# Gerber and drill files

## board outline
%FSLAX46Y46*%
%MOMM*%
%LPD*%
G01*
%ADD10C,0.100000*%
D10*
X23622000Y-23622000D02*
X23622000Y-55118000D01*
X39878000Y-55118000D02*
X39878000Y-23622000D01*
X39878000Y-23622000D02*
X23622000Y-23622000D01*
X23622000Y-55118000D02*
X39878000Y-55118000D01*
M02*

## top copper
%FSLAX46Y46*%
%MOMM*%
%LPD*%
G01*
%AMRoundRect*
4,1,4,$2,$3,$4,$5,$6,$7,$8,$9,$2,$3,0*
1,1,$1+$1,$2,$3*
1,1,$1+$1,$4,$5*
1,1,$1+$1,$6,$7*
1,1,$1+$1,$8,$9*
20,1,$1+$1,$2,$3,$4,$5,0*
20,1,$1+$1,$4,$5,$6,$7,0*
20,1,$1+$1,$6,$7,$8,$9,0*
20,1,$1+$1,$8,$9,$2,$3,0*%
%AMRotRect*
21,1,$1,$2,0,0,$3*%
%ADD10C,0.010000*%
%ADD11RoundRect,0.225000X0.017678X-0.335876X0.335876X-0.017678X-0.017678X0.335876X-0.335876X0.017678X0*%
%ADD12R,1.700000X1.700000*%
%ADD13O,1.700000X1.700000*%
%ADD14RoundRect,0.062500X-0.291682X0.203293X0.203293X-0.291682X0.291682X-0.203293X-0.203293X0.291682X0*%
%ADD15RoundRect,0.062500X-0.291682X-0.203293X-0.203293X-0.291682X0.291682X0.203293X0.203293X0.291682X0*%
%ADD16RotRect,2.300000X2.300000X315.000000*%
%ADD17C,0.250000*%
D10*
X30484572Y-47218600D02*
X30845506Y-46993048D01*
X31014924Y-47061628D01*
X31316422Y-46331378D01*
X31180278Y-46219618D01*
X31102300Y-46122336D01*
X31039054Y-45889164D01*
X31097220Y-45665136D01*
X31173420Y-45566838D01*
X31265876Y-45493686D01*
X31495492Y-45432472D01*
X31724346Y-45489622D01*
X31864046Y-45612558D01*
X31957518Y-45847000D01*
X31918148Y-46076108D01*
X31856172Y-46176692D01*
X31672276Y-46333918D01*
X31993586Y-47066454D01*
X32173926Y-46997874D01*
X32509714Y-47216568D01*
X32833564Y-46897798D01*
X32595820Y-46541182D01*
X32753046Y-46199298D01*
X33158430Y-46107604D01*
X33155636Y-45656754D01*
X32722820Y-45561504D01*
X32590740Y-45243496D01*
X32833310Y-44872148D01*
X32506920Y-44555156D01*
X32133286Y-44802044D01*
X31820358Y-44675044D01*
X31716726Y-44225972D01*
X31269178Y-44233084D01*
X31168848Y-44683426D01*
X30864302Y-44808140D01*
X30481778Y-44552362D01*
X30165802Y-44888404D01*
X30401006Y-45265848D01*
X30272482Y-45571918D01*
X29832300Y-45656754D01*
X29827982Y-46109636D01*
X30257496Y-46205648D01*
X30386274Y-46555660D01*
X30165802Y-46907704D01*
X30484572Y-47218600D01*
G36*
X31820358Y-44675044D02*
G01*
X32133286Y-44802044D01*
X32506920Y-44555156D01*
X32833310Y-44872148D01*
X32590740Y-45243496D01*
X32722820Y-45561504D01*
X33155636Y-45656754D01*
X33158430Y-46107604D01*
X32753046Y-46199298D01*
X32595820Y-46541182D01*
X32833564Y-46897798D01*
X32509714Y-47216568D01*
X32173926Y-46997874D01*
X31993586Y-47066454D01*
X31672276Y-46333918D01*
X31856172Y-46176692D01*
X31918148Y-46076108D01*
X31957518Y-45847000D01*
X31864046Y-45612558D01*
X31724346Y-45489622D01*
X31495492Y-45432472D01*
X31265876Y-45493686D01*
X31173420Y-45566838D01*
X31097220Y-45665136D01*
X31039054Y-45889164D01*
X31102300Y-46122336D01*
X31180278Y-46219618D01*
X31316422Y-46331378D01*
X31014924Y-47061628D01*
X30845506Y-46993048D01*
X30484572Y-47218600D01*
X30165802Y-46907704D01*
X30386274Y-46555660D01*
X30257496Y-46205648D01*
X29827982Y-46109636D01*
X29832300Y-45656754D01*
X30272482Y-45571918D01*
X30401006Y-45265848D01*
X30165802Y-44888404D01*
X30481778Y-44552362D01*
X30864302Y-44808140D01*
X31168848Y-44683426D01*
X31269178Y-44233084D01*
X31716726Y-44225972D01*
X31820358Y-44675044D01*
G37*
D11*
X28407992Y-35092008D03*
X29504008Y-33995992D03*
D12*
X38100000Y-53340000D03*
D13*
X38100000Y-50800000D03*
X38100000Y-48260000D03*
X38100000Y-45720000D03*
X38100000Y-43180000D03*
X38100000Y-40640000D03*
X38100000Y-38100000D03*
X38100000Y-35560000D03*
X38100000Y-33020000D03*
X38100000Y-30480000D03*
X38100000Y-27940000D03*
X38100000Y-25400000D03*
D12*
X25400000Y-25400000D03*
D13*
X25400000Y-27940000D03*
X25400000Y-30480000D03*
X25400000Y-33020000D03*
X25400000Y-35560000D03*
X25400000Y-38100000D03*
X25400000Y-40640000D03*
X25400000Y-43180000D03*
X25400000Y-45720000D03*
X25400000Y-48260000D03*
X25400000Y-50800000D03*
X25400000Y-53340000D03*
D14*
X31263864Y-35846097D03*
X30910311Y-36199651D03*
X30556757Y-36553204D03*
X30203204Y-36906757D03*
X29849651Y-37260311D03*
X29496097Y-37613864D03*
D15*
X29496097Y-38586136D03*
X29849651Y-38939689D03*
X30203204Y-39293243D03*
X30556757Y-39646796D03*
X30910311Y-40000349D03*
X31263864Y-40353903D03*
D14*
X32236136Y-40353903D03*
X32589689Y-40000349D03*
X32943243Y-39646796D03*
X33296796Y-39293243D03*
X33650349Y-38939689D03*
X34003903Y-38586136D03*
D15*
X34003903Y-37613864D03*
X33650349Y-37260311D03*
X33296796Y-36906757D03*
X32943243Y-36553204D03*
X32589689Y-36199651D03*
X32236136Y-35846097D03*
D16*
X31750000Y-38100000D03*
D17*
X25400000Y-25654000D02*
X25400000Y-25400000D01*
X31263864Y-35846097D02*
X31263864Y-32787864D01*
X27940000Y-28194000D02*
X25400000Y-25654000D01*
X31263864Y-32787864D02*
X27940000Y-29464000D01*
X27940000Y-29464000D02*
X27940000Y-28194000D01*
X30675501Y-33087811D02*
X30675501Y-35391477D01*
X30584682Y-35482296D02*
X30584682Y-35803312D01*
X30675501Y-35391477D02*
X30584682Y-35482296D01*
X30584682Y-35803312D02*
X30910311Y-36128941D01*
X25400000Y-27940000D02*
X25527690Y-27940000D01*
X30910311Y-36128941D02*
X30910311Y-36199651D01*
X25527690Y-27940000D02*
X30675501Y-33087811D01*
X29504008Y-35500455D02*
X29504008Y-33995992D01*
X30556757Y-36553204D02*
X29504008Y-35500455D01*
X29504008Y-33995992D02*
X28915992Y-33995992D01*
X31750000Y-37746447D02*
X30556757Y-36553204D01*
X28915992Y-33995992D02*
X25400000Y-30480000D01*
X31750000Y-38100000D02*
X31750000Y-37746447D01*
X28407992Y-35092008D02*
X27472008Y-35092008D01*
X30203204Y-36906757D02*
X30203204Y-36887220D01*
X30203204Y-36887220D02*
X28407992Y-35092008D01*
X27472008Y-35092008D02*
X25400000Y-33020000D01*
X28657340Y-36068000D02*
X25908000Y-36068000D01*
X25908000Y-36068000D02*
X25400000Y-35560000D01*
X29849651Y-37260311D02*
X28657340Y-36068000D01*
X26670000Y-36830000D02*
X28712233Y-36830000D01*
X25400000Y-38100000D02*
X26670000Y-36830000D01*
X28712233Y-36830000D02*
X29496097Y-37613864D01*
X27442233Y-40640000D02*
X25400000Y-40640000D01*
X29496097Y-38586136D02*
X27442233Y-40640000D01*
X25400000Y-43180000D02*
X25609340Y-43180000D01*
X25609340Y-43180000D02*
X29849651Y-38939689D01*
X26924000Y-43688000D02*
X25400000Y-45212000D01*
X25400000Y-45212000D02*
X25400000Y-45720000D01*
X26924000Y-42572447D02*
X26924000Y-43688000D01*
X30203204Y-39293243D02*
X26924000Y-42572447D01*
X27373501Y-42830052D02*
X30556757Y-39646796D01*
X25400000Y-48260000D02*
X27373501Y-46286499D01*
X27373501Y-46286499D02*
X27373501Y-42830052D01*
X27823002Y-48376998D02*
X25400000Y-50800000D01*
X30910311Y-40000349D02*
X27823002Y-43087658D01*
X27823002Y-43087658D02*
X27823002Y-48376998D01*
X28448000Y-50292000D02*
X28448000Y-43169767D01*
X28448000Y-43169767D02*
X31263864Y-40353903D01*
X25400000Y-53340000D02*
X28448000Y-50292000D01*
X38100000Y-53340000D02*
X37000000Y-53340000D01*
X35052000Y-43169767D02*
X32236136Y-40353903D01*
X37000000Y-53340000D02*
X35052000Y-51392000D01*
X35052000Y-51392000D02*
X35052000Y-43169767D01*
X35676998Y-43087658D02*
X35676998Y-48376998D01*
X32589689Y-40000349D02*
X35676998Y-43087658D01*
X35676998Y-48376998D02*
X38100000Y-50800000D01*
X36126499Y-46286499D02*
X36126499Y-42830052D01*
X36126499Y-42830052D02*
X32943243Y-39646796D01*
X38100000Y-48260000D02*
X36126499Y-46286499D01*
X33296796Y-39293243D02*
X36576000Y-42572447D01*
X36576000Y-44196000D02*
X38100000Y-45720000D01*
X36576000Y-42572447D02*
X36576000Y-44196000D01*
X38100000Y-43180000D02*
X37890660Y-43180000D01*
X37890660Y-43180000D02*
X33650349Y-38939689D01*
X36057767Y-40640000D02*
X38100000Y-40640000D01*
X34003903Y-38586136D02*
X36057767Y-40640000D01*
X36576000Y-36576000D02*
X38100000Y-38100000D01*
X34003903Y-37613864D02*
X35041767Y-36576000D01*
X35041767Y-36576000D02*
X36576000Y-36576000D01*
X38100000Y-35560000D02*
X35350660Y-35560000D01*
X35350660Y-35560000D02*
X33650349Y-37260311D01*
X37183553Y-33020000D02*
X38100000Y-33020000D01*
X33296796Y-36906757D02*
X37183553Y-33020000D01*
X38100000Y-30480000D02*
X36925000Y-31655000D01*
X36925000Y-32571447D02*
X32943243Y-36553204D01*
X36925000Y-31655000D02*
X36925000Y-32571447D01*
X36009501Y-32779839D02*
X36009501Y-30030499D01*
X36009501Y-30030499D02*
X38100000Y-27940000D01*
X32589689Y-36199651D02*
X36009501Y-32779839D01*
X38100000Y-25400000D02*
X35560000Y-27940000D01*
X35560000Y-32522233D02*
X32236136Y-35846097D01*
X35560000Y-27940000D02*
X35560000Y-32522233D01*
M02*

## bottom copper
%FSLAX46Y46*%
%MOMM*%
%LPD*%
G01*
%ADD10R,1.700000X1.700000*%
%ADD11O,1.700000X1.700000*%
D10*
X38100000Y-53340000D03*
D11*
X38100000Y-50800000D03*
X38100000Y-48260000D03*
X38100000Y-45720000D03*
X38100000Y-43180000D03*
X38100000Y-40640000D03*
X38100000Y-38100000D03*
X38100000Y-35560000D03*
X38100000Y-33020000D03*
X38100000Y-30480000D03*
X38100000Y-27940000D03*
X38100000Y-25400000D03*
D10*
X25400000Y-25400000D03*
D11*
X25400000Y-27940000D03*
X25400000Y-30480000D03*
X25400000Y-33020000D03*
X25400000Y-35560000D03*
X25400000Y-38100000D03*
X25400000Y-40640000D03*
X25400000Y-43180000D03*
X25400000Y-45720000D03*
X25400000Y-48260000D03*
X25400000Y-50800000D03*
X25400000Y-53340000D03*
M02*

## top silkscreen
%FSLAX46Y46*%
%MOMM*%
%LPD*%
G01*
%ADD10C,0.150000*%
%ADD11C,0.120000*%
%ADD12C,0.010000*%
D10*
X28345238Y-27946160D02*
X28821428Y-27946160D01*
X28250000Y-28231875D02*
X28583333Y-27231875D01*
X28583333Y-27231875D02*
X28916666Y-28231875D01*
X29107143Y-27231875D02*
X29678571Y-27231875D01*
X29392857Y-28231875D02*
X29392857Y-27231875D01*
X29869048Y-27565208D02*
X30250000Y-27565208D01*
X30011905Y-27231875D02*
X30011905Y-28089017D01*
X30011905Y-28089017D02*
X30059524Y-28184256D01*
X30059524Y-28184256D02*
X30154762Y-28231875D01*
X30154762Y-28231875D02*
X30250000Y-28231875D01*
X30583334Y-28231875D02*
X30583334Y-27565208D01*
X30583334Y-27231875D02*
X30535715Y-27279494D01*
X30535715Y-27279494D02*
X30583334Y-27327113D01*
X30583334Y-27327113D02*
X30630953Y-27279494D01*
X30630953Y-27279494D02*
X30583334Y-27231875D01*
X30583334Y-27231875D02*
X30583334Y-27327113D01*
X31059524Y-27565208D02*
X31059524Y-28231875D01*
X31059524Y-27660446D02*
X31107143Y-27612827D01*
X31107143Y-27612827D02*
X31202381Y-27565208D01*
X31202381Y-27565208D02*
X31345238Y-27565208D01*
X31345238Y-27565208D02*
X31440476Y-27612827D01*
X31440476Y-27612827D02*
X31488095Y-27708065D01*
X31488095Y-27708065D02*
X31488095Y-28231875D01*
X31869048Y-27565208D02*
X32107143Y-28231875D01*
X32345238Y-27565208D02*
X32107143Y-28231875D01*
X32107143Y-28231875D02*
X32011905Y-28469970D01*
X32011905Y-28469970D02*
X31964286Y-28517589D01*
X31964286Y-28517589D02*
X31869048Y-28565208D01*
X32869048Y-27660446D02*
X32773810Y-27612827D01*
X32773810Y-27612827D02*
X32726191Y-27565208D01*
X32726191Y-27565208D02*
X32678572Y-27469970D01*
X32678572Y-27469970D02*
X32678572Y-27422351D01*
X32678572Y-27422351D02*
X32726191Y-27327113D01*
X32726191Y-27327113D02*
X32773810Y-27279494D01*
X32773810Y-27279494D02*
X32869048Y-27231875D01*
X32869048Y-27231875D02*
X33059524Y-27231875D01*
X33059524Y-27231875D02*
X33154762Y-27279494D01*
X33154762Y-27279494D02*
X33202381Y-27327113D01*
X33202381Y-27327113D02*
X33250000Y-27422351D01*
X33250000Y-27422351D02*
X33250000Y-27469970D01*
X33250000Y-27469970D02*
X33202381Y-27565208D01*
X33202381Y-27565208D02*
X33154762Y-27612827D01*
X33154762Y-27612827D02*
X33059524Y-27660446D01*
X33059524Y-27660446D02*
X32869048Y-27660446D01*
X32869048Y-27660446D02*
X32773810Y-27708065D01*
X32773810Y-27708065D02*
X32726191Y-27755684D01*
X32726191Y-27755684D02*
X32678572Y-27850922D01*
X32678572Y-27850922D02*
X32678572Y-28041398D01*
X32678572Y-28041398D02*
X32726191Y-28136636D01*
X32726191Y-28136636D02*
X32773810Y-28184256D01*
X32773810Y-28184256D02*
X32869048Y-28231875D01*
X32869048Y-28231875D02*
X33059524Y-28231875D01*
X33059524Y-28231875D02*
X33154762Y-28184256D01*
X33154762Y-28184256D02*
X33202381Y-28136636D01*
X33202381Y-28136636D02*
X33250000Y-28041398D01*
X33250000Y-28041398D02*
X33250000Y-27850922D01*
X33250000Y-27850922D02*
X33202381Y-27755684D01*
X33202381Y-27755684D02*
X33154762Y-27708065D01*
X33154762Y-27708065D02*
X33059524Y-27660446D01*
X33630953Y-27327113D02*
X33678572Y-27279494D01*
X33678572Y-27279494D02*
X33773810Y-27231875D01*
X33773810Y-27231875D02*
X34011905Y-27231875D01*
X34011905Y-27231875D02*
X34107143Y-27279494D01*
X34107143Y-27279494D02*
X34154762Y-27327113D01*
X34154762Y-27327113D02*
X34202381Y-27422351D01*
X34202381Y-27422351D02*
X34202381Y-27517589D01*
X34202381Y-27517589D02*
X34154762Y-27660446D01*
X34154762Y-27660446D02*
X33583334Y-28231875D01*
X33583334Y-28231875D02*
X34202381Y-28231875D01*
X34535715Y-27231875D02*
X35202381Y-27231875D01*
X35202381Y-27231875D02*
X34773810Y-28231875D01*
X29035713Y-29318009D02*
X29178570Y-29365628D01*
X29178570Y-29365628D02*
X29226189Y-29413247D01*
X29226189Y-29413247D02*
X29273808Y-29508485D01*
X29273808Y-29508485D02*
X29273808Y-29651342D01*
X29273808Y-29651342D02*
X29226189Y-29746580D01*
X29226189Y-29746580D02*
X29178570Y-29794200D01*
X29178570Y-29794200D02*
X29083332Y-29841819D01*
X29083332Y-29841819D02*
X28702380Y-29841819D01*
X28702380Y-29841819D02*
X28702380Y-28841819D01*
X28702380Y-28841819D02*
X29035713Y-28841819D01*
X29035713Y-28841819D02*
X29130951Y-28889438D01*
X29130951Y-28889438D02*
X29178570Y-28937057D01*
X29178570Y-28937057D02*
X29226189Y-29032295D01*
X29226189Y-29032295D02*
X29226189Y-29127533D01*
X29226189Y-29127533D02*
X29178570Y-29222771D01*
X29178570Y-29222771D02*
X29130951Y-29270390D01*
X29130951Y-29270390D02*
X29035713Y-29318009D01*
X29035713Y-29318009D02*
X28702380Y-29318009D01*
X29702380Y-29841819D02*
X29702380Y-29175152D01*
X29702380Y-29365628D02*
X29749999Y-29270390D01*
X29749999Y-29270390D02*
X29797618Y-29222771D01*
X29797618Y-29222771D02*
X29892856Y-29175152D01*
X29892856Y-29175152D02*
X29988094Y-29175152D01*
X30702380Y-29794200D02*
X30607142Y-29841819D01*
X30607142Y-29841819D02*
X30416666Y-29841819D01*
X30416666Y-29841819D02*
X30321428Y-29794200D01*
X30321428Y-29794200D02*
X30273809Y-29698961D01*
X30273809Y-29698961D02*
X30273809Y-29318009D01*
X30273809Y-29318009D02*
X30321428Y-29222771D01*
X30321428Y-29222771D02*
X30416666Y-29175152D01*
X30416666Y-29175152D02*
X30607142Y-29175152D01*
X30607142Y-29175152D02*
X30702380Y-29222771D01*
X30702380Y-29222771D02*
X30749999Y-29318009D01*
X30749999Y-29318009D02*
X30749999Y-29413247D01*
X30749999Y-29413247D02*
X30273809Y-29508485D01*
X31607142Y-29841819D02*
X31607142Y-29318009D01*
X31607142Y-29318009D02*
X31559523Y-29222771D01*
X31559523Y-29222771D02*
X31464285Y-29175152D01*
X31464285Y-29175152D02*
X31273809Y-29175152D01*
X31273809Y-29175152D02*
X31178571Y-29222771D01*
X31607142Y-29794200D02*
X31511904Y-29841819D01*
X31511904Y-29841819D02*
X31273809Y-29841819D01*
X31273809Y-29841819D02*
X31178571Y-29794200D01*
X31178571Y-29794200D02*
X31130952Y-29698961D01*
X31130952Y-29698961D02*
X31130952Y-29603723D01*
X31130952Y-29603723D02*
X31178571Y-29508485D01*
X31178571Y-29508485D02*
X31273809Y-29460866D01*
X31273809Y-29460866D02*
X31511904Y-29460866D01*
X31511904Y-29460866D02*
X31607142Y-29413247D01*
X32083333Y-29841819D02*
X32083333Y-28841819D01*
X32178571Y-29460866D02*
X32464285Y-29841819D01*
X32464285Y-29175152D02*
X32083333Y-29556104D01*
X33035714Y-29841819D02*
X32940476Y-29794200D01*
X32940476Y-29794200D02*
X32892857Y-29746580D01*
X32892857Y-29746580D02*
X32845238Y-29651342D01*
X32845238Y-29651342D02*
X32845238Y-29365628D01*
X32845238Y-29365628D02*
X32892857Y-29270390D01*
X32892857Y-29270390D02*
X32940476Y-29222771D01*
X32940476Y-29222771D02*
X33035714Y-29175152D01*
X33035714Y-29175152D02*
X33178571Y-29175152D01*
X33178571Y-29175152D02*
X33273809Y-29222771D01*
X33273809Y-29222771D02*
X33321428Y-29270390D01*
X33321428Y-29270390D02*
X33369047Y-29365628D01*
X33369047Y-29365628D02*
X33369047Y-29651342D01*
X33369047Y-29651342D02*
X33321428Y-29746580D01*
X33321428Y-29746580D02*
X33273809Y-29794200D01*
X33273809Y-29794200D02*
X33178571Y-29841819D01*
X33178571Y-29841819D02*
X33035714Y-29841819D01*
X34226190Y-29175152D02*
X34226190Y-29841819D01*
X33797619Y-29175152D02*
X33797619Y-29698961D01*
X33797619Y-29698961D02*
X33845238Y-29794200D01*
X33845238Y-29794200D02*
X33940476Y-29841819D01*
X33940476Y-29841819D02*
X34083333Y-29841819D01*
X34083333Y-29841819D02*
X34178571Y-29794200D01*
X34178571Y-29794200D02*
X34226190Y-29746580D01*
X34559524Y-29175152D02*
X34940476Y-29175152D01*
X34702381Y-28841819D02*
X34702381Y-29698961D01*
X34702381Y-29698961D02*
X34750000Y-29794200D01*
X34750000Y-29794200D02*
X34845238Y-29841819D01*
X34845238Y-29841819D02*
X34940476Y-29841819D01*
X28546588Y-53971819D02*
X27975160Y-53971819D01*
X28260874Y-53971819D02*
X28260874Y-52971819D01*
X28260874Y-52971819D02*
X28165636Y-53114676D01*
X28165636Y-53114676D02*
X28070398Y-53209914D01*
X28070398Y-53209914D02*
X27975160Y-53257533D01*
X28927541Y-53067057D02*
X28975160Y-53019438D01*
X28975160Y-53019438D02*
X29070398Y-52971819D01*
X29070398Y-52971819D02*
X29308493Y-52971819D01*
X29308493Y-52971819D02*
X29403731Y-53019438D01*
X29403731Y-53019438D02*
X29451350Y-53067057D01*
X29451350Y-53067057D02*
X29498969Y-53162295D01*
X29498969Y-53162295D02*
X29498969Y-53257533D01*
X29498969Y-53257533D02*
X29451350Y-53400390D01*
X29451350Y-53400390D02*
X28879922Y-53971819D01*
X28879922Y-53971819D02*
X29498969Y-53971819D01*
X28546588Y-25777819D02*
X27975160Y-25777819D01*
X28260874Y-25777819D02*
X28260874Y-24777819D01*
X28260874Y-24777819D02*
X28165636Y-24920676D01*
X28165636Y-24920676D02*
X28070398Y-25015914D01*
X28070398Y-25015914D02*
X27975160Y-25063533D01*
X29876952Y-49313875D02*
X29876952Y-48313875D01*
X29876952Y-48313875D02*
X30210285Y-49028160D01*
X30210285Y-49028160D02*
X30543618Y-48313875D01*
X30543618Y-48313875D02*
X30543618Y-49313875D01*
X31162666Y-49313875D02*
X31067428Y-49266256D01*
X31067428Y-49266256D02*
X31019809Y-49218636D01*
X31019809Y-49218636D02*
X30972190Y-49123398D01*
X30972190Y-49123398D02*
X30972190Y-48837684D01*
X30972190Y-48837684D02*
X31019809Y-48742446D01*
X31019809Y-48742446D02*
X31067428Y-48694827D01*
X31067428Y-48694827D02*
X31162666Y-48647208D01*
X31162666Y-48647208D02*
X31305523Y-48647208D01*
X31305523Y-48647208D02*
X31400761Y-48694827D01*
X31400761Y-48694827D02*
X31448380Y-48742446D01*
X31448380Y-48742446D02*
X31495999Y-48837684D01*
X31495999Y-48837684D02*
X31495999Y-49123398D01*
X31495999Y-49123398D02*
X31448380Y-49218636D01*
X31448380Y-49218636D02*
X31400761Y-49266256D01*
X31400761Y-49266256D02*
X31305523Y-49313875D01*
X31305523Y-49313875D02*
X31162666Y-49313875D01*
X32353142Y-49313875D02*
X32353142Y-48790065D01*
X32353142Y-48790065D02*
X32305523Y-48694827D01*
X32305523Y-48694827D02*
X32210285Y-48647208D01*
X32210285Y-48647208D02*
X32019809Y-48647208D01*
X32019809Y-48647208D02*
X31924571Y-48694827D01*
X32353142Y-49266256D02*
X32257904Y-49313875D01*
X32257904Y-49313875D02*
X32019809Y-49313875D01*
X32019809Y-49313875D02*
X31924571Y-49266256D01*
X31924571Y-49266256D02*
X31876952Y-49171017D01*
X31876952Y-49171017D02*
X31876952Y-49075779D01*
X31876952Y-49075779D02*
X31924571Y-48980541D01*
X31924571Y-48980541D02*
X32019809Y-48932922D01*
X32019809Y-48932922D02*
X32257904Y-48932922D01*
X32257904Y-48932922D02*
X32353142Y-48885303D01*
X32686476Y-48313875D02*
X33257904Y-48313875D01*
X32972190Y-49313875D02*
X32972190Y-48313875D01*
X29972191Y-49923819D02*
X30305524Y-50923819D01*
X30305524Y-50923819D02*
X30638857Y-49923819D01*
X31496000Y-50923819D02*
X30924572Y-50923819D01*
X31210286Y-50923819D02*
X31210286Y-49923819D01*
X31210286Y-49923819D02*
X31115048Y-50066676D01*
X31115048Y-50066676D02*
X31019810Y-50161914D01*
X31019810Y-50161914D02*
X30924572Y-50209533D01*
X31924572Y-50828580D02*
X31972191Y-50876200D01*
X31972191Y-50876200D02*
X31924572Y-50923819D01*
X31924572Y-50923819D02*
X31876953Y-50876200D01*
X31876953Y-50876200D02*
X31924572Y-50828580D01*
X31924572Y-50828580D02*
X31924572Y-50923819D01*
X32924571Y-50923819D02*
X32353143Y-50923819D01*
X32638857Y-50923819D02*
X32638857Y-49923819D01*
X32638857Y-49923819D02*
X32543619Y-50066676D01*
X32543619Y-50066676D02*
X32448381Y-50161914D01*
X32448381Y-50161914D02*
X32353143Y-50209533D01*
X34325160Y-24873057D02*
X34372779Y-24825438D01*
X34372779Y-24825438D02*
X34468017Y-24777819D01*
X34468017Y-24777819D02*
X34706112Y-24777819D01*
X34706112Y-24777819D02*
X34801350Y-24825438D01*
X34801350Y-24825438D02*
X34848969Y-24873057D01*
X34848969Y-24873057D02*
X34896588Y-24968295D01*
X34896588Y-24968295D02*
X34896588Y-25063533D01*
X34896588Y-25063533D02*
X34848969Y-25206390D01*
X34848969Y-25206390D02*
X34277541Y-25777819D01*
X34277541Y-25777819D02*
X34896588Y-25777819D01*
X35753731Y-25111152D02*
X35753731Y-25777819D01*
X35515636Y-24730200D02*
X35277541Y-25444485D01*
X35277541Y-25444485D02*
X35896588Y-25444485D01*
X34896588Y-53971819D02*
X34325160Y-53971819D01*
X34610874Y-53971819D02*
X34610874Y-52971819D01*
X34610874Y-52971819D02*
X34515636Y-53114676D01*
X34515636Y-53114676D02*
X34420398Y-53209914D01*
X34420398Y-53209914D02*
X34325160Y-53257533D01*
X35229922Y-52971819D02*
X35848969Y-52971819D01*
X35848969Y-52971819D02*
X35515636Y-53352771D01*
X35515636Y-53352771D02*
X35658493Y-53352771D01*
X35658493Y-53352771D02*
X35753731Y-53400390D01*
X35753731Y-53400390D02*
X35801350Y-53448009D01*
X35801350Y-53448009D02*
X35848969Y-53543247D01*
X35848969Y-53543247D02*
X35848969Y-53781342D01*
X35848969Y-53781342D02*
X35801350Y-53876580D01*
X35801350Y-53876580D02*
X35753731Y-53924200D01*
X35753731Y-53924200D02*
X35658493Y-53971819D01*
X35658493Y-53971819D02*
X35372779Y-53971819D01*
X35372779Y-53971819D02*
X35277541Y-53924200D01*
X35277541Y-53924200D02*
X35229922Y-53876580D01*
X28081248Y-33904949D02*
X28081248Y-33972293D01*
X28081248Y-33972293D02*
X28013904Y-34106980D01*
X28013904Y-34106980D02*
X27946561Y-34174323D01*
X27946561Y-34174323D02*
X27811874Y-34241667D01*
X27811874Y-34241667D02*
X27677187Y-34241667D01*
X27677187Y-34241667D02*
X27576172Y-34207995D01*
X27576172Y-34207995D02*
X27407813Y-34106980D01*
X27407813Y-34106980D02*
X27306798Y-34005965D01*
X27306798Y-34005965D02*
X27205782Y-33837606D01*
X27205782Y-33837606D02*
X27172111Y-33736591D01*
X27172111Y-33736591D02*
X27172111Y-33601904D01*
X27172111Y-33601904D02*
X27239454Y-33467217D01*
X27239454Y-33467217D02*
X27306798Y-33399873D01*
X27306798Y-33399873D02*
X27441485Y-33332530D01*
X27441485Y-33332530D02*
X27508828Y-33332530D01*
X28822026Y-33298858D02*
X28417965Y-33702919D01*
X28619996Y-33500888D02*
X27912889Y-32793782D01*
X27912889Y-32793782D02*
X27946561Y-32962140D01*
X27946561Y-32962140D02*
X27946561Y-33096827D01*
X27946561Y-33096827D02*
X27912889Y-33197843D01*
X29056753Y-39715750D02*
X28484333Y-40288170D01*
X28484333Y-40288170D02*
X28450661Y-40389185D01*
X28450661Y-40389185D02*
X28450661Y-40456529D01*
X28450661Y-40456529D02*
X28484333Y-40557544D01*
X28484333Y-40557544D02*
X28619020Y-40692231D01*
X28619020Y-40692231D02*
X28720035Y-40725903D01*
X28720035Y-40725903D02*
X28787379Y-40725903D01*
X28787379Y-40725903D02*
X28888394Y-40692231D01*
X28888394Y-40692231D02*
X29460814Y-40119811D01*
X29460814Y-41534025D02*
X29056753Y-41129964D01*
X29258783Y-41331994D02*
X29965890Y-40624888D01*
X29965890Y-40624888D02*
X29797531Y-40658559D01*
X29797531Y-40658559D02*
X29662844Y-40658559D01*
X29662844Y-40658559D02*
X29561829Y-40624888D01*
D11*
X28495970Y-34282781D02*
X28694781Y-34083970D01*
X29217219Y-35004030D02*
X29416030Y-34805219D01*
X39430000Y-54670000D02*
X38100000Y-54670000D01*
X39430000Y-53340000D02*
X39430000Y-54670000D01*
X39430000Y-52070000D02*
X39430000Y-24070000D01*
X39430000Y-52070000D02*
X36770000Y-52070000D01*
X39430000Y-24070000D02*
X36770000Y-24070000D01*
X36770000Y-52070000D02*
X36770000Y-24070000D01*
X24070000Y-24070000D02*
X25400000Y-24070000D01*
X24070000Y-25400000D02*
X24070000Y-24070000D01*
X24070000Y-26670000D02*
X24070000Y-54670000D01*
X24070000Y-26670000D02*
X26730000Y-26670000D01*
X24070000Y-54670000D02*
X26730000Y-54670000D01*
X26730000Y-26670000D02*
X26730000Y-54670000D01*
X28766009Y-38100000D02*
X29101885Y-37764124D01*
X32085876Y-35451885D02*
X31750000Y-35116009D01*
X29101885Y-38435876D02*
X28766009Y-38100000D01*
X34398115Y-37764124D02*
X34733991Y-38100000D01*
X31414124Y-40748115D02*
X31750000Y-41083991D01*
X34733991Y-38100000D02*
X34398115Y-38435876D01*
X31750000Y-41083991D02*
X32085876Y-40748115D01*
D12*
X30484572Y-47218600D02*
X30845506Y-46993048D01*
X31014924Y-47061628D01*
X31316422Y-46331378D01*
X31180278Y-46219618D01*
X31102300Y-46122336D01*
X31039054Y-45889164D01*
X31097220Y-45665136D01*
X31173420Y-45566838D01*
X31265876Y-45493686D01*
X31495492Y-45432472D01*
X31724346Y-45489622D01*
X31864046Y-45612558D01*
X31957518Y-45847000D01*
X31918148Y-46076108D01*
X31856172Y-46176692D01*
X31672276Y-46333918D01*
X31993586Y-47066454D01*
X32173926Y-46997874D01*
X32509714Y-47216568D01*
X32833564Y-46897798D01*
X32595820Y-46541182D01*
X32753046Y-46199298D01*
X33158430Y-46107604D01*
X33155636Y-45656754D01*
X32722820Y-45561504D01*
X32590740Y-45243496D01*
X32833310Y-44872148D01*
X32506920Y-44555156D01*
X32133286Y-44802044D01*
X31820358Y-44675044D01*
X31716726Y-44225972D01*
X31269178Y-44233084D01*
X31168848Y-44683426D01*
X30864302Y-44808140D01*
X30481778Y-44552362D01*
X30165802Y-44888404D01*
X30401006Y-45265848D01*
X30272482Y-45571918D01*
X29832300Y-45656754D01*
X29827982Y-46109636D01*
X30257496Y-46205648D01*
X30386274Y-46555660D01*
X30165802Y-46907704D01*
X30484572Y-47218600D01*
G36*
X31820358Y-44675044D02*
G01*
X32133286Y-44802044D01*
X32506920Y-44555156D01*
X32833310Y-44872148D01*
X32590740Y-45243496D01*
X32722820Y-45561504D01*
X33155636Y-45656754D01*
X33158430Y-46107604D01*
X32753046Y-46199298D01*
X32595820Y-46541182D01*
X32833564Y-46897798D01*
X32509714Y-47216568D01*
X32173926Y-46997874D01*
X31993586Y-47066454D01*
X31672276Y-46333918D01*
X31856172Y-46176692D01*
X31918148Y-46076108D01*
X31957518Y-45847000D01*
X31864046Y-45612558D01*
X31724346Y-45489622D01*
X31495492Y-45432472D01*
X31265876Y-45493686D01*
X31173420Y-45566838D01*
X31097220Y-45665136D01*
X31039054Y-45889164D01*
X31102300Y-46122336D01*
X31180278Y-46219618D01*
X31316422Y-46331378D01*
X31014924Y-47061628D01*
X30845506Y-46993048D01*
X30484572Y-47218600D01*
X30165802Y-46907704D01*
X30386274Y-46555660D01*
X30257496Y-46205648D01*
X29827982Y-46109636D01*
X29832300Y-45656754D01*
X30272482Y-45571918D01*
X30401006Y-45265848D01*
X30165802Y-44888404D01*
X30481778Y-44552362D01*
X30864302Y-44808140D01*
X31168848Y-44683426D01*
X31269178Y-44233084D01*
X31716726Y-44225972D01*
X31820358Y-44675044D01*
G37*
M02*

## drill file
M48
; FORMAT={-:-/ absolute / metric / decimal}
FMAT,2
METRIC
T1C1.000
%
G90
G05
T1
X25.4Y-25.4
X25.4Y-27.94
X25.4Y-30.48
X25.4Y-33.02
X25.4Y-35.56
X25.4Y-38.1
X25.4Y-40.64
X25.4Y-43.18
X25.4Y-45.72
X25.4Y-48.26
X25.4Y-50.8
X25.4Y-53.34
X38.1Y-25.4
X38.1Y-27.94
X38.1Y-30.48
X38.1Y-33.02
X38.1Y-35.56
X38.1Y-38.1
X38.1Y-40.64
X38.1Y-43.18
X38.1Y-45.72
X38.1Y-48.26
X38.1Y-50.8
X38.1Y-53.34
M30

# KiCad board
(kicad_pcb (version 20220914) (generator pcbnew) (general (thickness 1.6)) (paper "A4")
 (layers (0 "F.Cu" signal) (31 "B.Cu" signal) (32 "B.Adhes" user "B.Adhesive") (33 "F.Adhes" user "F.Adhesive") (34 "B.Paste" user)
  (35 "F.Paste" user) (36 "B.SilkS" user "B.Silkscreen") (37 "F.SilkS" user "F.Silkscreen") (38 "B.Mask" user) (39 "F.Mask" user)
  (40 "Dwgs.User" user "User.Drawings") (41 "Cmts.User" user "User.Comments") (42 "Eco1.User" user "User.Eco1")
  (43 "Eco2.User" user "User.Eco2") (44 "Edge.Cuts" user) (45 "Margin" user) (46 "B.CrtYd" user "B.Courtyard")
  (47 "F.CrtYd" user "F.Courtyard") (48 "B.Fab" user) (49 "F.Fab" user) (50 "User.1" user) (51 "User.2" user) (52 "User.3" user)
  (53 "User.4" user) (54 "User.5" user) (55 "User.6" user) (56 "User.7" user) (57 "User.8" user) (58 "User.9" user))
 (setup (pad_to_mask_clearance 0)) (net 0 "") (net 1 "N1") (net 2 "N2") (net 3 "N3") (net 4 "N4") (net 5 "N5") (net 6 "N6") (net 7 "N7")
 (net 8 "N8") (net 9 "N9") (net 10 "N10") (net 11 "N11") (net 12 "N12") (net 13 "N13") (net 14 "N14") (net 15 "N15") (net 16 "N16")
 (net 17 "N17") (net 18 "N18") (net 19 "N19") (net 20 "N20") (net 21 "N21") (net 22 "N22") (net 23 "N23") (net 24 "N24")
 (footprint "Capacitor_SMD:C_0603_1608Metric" (layer "F.Cu") (at 28.956 34.544 45)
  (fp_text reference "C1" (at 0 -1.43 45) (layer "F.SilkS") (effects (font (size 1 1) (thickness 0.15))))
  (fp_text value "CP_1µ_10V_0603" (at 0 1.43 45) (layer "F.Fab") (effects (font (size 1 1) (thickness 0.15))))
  (fp_line (start -0.14058 -0.51) (end 0.14058 -0.51) (stroke (width 0.12) (type solid)) (layer "F.SilkS"))
  (fp_line (start -0.14058 0.51) (end 0.14058 0.51) (stroke (width 0.12) (type solid)) (layer "F.SilkS"))
  (pad "1" smd roundrect (at -0.775 0 45) (size 0.9 0.95) (layers "F.Cu" "F.Paste" "F.Mask") (roundrect_rratio 0.25) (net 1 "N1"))
  (pad "2" smd roundrect (at 0.775 0 45) (size 0.9 0.95) (layers "F.Cu" "F.Paste" "F.Mask") (roundrect_rratio 0.25) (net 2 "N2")))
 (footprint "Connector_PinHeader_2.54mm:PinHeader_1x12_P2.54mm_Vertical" (layer "F.Cu") (at 38.1 53.34 180)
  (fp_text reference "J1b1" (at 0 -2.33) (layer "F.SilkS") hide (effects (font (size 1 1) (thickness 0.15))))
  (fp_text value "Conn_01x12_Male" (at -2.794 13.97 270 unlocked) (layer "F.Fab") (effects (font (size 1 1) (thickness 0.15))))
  (fp_line (start -1.33 -1.33) (end 0 -1.33) (stroke (width 0.12) (type solid)) (layer "F.SilkS"))
  (fp_line (start -1.33 0) (end -1.33 -1.33) (stroke (width 0.12) (type solid)) (layer "F.SilkS"))
  (fp_line (start -1.33 1.27) (end -1.33 29.27) (stroke (width 0.12) (type solid)) (layer "F.SilkS"))
  (fp_line (start -1.33 1.27) (end 1.33 1.27) (stroke (width 0.12) (type solid)) (layer "F.SilkS"))
  (fp_line (start -1.33 29.27) (end 1.33 29.27) (stroke (width 0.12) (type solid)) (layer "F.SilkS"))
  (fp_line (start 1.33 1.27) (end 1.33 29.27) (stroke (width 0.12) (type solid)) (layer "F.SilkS"))
  (pad "1" thru_hole rect (at 0 0 180) (size 1.7 1.7) (drill 1) (layers *.Cu *.Mask) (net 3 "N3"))
  (pad "2" thru_hole oval (at 0 2.54 180) (size 1.7 1.7) (drill 1) (layers *.Cu *.Mask) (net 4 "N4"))
  (pad "3" thru_hole oval (at 0 5.08 180) (size 1.7 1.7) (drill 1) (layers *.Cu *.Mask) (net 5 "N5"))
  (pad "4" thru_hole oval (at 0 7.62 180) (size 1.7 1.7) (drill 1) (layers *.Cu *.Mask) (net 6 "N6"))
  (pad "5" thru_hole oval (at 0 10.16 180) (size 1.7 1.7) (drill 1) (layers *.Cu *.Mask) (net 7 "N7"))
  (pad "6" thru_hole oval (at 0 12.7 180) (size 1.7 1.7) (drill 1) (layers *.Cu *.Mask) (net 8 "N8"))
  (pad "7" thru_hole oval (at 0 15.24 180) (size 1.7 1.7) (drill 1) (layers *.Cu *.Mask) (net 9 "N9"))
  (pad "8" thru_hole oval (at 0 17.78 180) (size 1.7 1.7) (drill 1) (layers *.Cu *.Mask) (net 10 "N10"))
  (pad "9" thru_hole oval (at 0 20.32 180) (size 1.7 1.7) (drill 1) (layers *.Cu *.Mask) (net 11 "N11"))
  (pad "10" thru_hole oval (at 0 22.86 180) (size 1.7 1.7) (drill 1) (layers *.Cu *.Mask) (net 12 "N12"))
  (pad "11" thru_hole oval (at 0 25.4 180) (size 1.7 1.7) (drill 1) (layers *.Cu *.Mask) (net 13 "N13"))
  (pad "12" thru_hole oval (at 0 27.94 180) (size 1.7 1.7) (drill 1) (layers *.Cu *.Mask) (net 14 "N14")))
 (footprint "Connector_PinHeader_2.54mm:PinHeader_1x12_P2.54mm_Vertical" (layer "F.Cu") (at 25.4 25.4)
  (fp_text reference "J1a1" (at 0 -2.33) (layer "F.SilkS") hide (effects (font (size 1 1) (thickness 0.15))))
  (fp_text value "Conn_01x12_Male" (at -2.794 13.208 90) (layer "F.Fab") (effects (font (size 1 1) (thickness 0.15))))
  (fp_line (start -1.33 -1.33) (end 0 -1.33) (stroke (width 0.12) (type solid)) (layer "F.SilkS"))
  (fp_line (start -1.33 0) (end -1.33 -1.33) (stroke (width 0.12) (type solid)) (layer "F.SilkS"))
  (fp_line (start -1.33 1.27) (end -1.33 29.27) (stroke (width 0.12) (type solid)) (layer "F.SilkS"))
  (fp_line (start -1.33 1.27) (end 1.33 1.27) (stroke (width 0.12) (type solid)) (layer "F.SilkS"))
  (fp_line (start -1.33 29.27) (end 1.33 29.27) (stroke (width 0.12) (type solid)) (layer "F.SilkS"))
  (fp_line (start 1.33 1.27) (end 1.33 29.27) (stroke (width 0.12) (type solid)) (layer "F.SilkS"))
  (pad "1" thru_hole rect (at 0 0) (size 1.7 1.7) (drill 1) (layers *.Cu *.Mask) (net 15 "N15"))
  (pad "2" thru_hole oval (at 0 2.54) (size 1.7 1.7) (drill 1) (layers *.Cu *.Mask) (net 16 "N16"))
  (pad "3" thru_hole oval (at 0 5.08) (size 1.7 1.7) (drill 1) (layers *.Cu *.Mask) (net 2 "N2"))
  (pad "4" thru_hole oval (at 0 7.62) (size 1.7 1.7) (drill 1) (layers *.Cu *.Mask) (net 1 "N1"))
  (pad "5" thru_hole oval (at 0 10.16) (size 1.7 1.7) (drill 1) (layers *.Cu *.Mask) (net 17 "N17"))
  (pad "6" thru_hole oval (at 0 12.7) (size 1.7 1.7) (drill 1) (layers *.Cu *.Mask) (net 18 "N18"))
  (pad "7" thru_hole oval (at 0 15.24) (size 1.7 1.7) (drill 1) (layers *.Cu *.Mask) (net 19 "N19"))
  (pad "8" thru_hole oval (at 0 17.78) (size 1.7 1.7) (drill 1) (layers *.Cu *.Mask) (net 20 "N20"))
  (pad "9" thru_hole oval (at 0 20.32) (size 1.7 1.7) (drill 1) (layers *.Cu *.Mask) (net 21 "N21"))
  (pad "10" thru_hole oval (at 0 22.86) (size 1.7 1.7) (drill 1) (layers *.Cu *.Mask) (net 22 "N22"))
  (pad "11" thru_hole oval (at 0 25.4) (size 1.7 1.7) (drill 1) (layers *.Cu *.Mask) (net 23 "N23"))
  (pad "12" thru_hole oval (at 0 27.94) (size 1.7 1.7) (drill 1) (layers *.Cu *.Mask) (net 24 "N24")))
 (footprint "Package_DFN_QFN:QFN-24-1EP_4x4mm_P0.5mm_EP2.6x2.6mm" (layer "F.Cu") (at 31.75 38.1 -45)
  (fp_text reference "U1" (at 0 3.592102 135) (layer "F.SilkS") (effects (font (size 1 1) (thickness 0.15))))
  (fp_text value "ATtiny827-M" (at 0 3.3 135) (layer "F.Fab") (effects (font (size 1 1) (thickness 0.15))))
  (fp_line (start -2.11 2.11) (end -2.11 1.635) (stroke (width 0.12) (type solid)) (layer "F.SilkS"))
  (fp_line (start -1.635 -2.11) (end -2.11 -2.11) (stroke (width 0.12) (type solid)) (layer "F.SilkS"))
  (fp_line (start -1.635 2.11) (end -2.11 2.11) (stroke (width 0.12) (type solid)) (layer "F.SilkS"))
  (fp_line (start 1.635 -2.11) (end 2.11 -2.11) (stroke (width 0.12) (type solid)) (layer "F.SilkS"))
  (fp_line (start 1.635 2.11) (end 2.11 2.11) (stroke (width 0.12) (type solid)) (layer "F.SilkS"))
  (fp_line (start 2.11 -2.11) (end 2.11 -1.635) (stroke (width 0.12) (type solid)) (layer "F.SilkS"))
  (fp_line (start 2.11 2.11) (end 2.11 1.635) (stroke (width 0.12) (type solid)) (layer "F.SilkS"))
  (pad "" smd roundrect (at -0.65 -0.65 315) (size 1.05 1.05) (layers "F.Paste") (roundrect_rratio 0.2380952381))
  (pad "" smd roundrect (at -0.65 0.65 315) (size 1.05 1.05) (layers "F.Paste") (roundrect_rratio 0.2380952381))
  (pad "" smd roundrect (at 0.65 -0.65 315) (size 1.05 1.05) (layers "F.Paste") (roundrect_rratio 0.2380952381))
  (pad "" smd roundrect (at 0.65 0.65 315) (size 1.05 1.05) (layers "F.Paste") (roundrect_rratio 0.2380952381))
  (pad "1" smd roundrect (at -1.9375 -1.25 315) (size 0.825 0.25) (layers "F.Cu" "F.Paste" "F.Mask") (roundrect_rratio 0.25) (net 15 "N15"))
  (pad "2" smd roundrect (at -1.9375 -0.75 315) (size 0.825 0.25) (layers "F.Cu" "F.Paste" "F.Mask") (roundrect_rratio 0.25) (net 16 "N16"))
  (pad "3" smd roundrect (at -1.9375 -0.25 315) (size 0.825 0.25) (layers "F.Cu" "F.Paste" "F.Mask") (roundrect_rratio 0.25) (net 2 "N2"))
  (pad "4" smd roundrect (at -1.9375 0.25 315) (size 0.825 0.25) (layers "F.Cu" "F.Paste" "F.Mask") (roundrect_rratio 0.25) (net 1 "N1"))
  (pad "5" smd roundrect (at -1.9375 0.75 315) (size 0.825 0.25) (layers "F.Cu" "F.Paste" "F.Mask") (roundrect_rratio 0.25) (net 17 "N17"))
  (pad "6" smd roundrect (at -1.9375 1.25 315) (size 0.825 0.25) (layers "F.Cu" "F.Paste" "F.Mask") (roundrect_rratio 0.25) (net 18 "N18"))
  (pad "7" smd roundrect (at -1.25 1.9375 315) (size 0.25 0.825) (layers "F.Cu" "F.Paste" "F.Mask") (roundrect_rratio 0.25) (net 19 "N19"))
  (pad "8" smd roundrect (at -0.75 1.9375 315) (size 0.25 0.825) (layers "F.Cu" "F.Paste" "F.Mask") (roundrect_rratio 0.25) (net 20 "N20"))
  (pad "9" smd roundrect (at -0.25 1.9375 315) (size 0.25 0.825) (layers "F.Cu" "F.Paste" "F.Mask") (roundrect_rratio 0.25) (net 21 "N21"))
  (pad "10" smd roundrect (at 0.25 1.9375 315) (size 0.25 0.825) (layers "F.Cu" "F.Paste" "F.Mask") (roundrect_rratio 0.25) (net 22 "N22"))
  (pad "11" smd roundrect (at 0.75 1.9375 315) (size 0.25 0.825) (layers "F.Cu" "F.Paste" "F.Mask") (roundrect_rratio 0.25) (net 23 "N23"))
  (pad "12" smd roundrect (at 1.25 1.9375 315) (size 0.25 0.825) (layers "F.Cu" "F.Paste" "F.Mask") (roundrect_rratio 0.25) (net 24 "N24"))
  (pad "13" smd roundrect (at 1.9375 1.25 315) (size 0.825 0.25) (layers "F.Cu" "F.Paste" "F.Mask") (roundrect_rratio 0.25) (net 3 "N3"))
  (pad "14" smd roundrect (at 1.9375 0.75 315) (size 0.825 0.25) (layers "F.Cu" "F.Paste" "F.Mask") (roundrect_rratio 0.25) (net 4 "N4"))
  (pad "15" smd roundrect (at 1.9375 0.25 315) (size 0.825 0.25) (layers "F.Cu" "F.Paste" "F.Mask") (roundrect_rratio 0.25) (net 5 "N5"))
  (pad "16" smd roundrect (at 1.9375 -0.25 315) (size 0.825 0.25) (layers "F.Cu" "F.Paste" "F.Mask") (roundrect_rratio 0.25) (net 6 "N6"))
  (pad "17" smd roundrect (at 1.9375 -0.75 315) (size 0.825 0.25) (layers "F.Cu" "F.Paste" "F.Mask") (roundrect_rratio 0.25) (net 7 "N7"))
  (pad "18" smd roundrect (at 1.9375 -1.25 315) (size 0.825 0.25) (layers "F.Cu" "F.Paste" "F.Mask") (roundrect_rratio 0.25) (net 8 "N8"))
  (pad "19" smd roundrect (at 1.25 -1.9375 315) (size 0.25 0.825) (layers "F.Cu" "F.Paste" "F.Mask") (roundrect_rratio 0.25) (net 9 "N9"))
  (pad "20" smd roundrect (at 0.75 -1.9375 315) (size 0.25 0.825) (layers "F.Cu" "F.Paste" "F.Mask") (roundrect_rratio 0.25) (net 10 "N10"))
  (pad "21" smd roundrect (at 0.25 -1.9375 315) (size 0.25 0.825) (layers "F.Cu" "F.Paste" "F.Mask") (roundrect_rratio 0.25) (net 11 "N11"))
  (pad "22" smd roundrect (at -0.25 -1.9375 315) (size 0.25 0.825) (layers "F.Cu" "F.Paste" "F.Mask") (roundrect_rratio 0.25) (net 12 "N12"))
  (pad "23" smd roundrect (at -0.75 -1.9375 315) (size 0.25 0.825) (layers "F.Cu" "F.Paste" "F.Mask") (roundrect_rratio 0.25) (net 13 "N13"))
  (pad "24" smd roundrect (at -1.25 -1.9375 315) (size 0.25 0.825) (layers "F.Cu" "F.Paste" "F.Mask") (roundrect_rratio 0.25) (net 14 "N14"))
  (pad "25" smd rect (at 0 0 315) (size 2.3 2.3) (layers "F.Cu" "F.Mask") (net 2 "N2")))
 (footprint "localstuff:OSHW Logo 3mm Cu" (layer "F.Cu") (at 31.496 45.72)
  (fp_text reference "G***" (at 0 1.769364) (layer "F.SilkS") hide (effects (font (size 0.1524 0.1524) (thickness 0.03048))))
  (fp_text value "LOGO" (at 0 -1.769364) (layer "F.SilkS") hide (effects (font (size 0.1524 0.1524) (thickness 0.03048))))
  (fp_poly
   (pts (xy -1.011428 1.4986) (xy -0.650494 1.273048) (xy -0.481076 1.341628) (xy -0.179578 0.611378) (xy -0.315722 0.499618)
    (xy -0.3937 0.402336) (xy -0.456946 0.169164) (xy -0.39878 -0.054864) (xy -0.32258 -0.153162) (xy -0.230124 -0.226314)
    (xy -0.000508 -0.287528) (xy 0.228346 -0.230378) (xy 0.368046 -0.107442) (xy 0.461518 0.127) (xy 0.422148 0.356108)
    (xy 0.360172 0.456692) (xy 0.176276 0.613918) (xy 0.497586 1.346454) (xy 0.677926 1.277874) (xy 1.013714 1.496568)
    (xy 1.337564 1.177798) (xy 1.09982 0.821182) (xy 1.257046 0.479298) (xy 1.66243 0.387604) (xy 1.659636 -0.063246) (xy 1.22682 -0.158496)
    (xy 1.09474 -0.476504) (xy 1.33731 -0.847852) (xy 1.01092 -1.164844) (xy 0.637286 -0.917956) (xy 0.324358 -1.044956)
    (xy 0.220726 -1.494028) (xy -0.226822 -1.486916) (xy -0.327152 -1.036574) (xy -0.631698 -0.91186) (xy -1.014222 -1.167638)
    (xy -1.330198 -0.831596) (xy -1.094994 -0.454152) (xy -1.223518 -0.148082) (xy -1.6637 -0.063246) (xy -1.668018 0.389636)
    (xy -1.238504 0.485648) (xy -1.109726 0.83566) (xy -1.330198 1.187704) (xy -1.011428 1.4986))
   (stroke (width 0.01) (type solid)) (fill solid) (layer "F.Cu")))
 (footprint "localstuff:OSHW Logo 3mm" (layer "F.Cu") (at 31.496 45.72)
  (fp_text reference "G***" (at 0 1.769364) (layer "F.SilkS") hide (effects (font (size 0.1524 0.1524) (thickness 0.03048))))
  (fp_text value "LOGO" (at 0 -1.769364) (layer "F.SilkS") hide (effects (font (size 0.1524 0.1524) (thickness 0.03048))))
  (fp_poly
   (pts (xy -1.011428 1.4986) (xy -0.650494 1.273048) (xy -0.481076 1.341628) (xy -0.179578 0.611378) (xy -0.315722 0.499618)
    (xy -0.3937 0.402336) (xy -0.456946 0.169164) (xy -0.39878 -0.054864) (xy -0.32258 -0.153162) (xy -0.230124 -0.226314)
    (xy -0.000508 -0.287528) (xy 0.228346 -0.230378) (xy 0.368046 -0.107442) (xy 0.461518 0.127) (xy 0.422148 0.356108)
    (xy 0.360172 0.456692) (xy 0.176276 0.613918) (xy 0.497586 1.346454) (xy 0.677926 1.277874) (xy 1.013714 1.496568)
    (xy 1.337564 1.177798) (xy 1.09982 0.821182) (xy 1.257046 0.479298) (xy 1.66243 0.387604) (xy 1.659636 -0.063246) (xy 1.22682 -0.158496)
    (xy 1.09474 -0.476504) (xy 1.33731 -0.847852) (xy 1.01092 -1.164844) (xy 0.637286 -0.917956) (xy 0.324358 -1.044956)
    (xy 0.220726 -1.494028) (xy -0.226822 -1.486916) (xy -0.327152 -1.036574) (xy -0.631698 -0.91186) (xy -1.014222 -1.167638)
    (xy -1.330198 -0.831596) (xy -1.094994 -0.454152) (xy -1.223518 -0.148082) (xy -1.6637 -0.063246) (xy -1.668018 0.389636)
    (xy -1.238504 0.485648) (xy -1.109726 0.83566) (xy -1.330198 1.187704) (xy -1.011428 1.4986))
   (stroke (width 0.01) (type solid)) (fill solid) (layer "F.SilkS")))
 (gr_line (start 23.622 23.622) (end 23.622 55.118) (stroke (width 0.1) (type default)) (layer "Edge.Cuts"))
 (gr_line (start 39.878 55.118) (end 39.878 23.622) (stroke (width 0.1) (type default)) (layer "Edge.Cuts"))
 (gr_line (start 39.878 23.622) (end 23.622 23.622) (stroke (width 0.1) (type default)) (layer "Edge.Cuts"))
 (gr_line (start 23.622 55.118) (end 39.878 55.118) (stroke (width 0.1) (type default)) (layer "Edge.Cuts"))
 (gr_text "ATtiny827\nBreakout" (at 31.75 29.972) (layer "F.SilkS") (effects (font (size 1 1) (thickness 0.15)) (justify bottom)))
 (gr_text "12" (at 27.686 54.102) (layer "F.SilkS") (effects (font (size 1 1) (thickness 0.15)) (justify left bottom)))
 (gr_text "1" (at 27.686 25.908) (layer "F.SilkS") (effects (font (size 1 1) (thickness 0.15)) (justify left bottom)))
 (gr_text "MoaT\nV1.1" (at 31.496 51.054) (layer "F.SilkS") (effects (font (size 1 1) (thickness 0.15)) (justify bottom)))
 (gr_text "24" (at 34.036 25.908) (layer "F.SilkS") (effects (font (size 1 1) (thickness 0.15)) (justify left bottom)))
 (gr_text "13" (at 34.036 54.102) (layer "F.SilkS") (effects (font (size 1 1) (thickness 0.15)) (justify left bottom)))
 (segment (start 25.4 25.654) (end 25.4 25.4) (width 0.25) (layer "F.Cu") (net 15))
 (segment (start 31.263864 35.846097) (end 31.263864 32.787864) (width 0.25) (layer "F.Cu") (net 15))
 (segment (start 27.94 28.194) (end 25.4 25.654) (width 0.25) (layer "F.Cu") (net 15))
 (segment (start 31.263864 32.787864) (end 27.94 29.464) (width 0.25) (layer "F.Cu") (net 15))
 (segment (start 27.94 29.464) (end 27.94 28.194) (width 0.25) (layer "F.Cu") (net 15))
 (segment (start 30.675501 33.087811) (end 30.675501 35.391477) (width 0.25) (layer "F.Cu") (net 16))
 (segment (start 30.584682 35.482296) (end 30.584682 35.803312) (width 0.25) (layer "F.Cu") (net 16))
 (segment (start 30.675501 35.391477) (end 30.584682 35.482296) (width 0.25) (layer "F.Cu") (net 16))
 (segment (start 30.584682 35.803312) (end 30.910311 36.128941) (width 0.25) (layer "F.Cu") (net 16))
 (segment (start 25.4 27.94) (end 25.52769 27.94) (width 0.25) (layer "F.Cu") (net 16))
 (segment (start 30.910311 36.128941) (end 30.910311 36.199651) (width 0.25) (layer "F.Cu") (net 16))
 (segment (start 25.52769 27.94) (end 30.675501 33.087811) (width 0.25) (layer "F.Cu") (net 16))
 (segment (start 29.504008 35.500455) (end 29.504008 33.995992) (width 0.25) (layer "F.Cu") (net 2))
 (segment (start 30.556757 36.553204) (end 29.504008 35.500455) (width 0.25) (layer "F.Cu") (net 2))
 (segment (start 29.504008 33.995992) (end 28.915992 33.995992) (width 0.25) (layer "F.Cu") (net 2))
 (segment (start 31.75 37.746447) (end 30.556757 36.553204) (width 0.25) (layer "F.Cu") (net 2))
 (segment (start 28.915992 33.995992) (end 25.4 30.48) (width 0.25) (layer "F.Cu") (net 2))
 (segment (start 31.75 38.1) (end 31.75 37.746447) (width 0.25) (layer "F.Cu") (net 2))
 (segment (start 28.407992 35.092008) (end 27.472008 35.092008) (width 0.25) (layer "F.Cu") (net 1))
 (segment (start 30.203204 36.906757) (end 30.203204 36.88722) (width 0.25) (layer "F.Cu") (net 1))
 (segment (start 30.203204 36.88722) (end 28.407992 35.092008) (width 0.25) (layer "F.Cu") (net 1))
 (segment (start 27.472008 35.092008) (end 25.4 33.02) (width 0.25) (layer "F.Cu") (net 1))
 (segment (start 28.65734 36.068) (end 25.908 36.068) (width 0.25) (layer "F.Cu") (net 17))
 (segment (start 25.908 36.068) (end 25.4 35.56) (width 0.25) (layer "F.Cu") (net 17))
 (segment (start 29.849651 37.260311) (end 28.65734 36.068) (width 0.25) (layer "F.Cu") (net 17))
 (segment (start 26.67 36.83) (end 28.712233 36.83) (width 0.25) (layer "F.Cu") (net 18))
 (segment (start 25.4 38.1) (end 26.67 36.83) (width 0.25) (layer "F.Cu") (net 18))
 (segment (start 28.712233 36.83) (end 29.496097 37.613864) (width 0.25) (layer "F.Cu") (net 18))
 (segment (start 27.442233 40.64) (end 25.4 40.64) (width 0.25) (layer "F.Cu") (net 19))
 (segment (start 29.496097 38.586136) (end 27.442233 40.64) (width 0.25) (layer "F.Cu") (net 19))
 (segment (start 25.4 43.18) (end 25.60934 43.18) (width 0.25) (layer "F.Cu") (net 20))
 (segment (start 25.60934 43.18) (end 29.849651 38.939689) (width 0.25) (layer "F.Cu") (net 20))
 (segment (start 26.924 43.688) (end 25.4 45.212) (width 0.25) (layer "F.Cu") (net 21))
 (segment (start 25.4 45.212) (end 25.4 45.72) (width 0.25) (layer "F.Cu") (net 21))
 (segment (start 26.924 42.572447) (end 26.924 43.688) (width 0.25) (layer "F.Cu") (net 21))
 (segment (start 30.203204 39.293243) (end 26.924 42.572447) (width 0.25) (layer "F.Cu") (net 21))
 (segment (start 27.373501 42.830052) (end 30.556757 39.646796) (width 0.25) (layer "F.Cu") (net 22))
 (segment (start 25.4 48.26) (end 27.373501 46.286499) (width 0.25) (layer "F.Cu") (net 22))
 (segment (start 27.373501 46.286499) (end 27.373501 42.830052) (width 0.25) (layer "F.Cu") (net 22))
 (segment (start 27.823002 48.376998) (end 25.4 50.8) (width 0.25) (layer "F.Cu") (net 23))
 (segment (start 30.910311 40.000349) (end 27.823002 43.087658) (width 0.25) (layer "F.Cu") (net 23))
 (segment (start 27.823002 43.087658) (end 27.823002 48.376998) (width 0.25) (layer "F.Cu") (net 23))
 (segment (start 28.448 50.292) (end 28.448 43.169767) (width 0.25) (layer "F.Cu") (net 24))
 (segment (start 28.448 43.169767) (end 31.263864 40.353903) (width 0.25) (layer "F.Cu") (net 24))
 (segment (start 25.4 53.34) (end 28.448 50.292) (width 0.25) (layer "F.Cu") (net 24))
 (segment (start 38.1 53.34) (end 37 53.34) (width 0.25) (layer "F.Cu") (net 3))
 (segment (start 35.052 43.169767) (end 32.236136 40.353903) (width 0.25) (layer "F.Cu") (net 3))
 (segment (start 37 53.34) (end 35.052 51.392) (width 0.25) (layer "F.Cu") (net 3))
 (segment (start 35.052 51.392) (end 35.052 43.169767) (width 0.25) (layer "F.Cu") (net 3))
 (segment (start 35.676998 43.087658) (end 35.676998 48.376998) (width 0.25) (layer "F.Cu") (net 4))
 (segment (start 32.589689 40.000349) (end 35.676998 43.087658) (width 0.25) (layer "F.Cu") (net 4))
 (segment (start 35.676998 48.376998) (end 38.1 50.8) (width 0.25) (layer "F.Cu") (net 4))
 (segment (start 36.126499 46.286499) (end 36.126499 42.830052) (width 0.25) (layer "F.Cu") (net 5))
 (segment (start 36.126499 42.830052) (end 32.943243 39.646796) (width 0.25) (layer "F.Cu") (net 5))
 (segment (start 38.1 48.26) (end 36.126499 46.286499) (width 0.25) (layer "F.Cu") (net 5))
 (segment (start 33.296796 39.293243) (end 36.576 42.572447) (width 0.25) (layer "F.Cu") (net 6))
 (segment (start 36.576 44.196) (end 38.1 45.72) (width 0.25) (layer "F.Cu") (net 6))
 (segment (start 36.576 42.572447) (end 36.576 44.196) (width 0.25) (layer "F.Cu") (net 6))
 (segment (start 38.1 43.18) (end 37.89066 43.18) (width 0.25) (layer "F.Cu") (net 7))
 (segment (start 37.89066 43.18) (end 33.650349 38.939689) (width 0.25) (layer "F.Cu") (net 7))
 (segment (start 36.057767 40.64) (end 38.1 40.64) (width 0.25) (layer "F.Cu") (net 8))
 (segment (start 34.003903 38.586136) (end 36.057767 40.64) (width 0.25) (layer "F.Cu") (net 8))
 (segment (start 36.576 36.576) (end 38.1 38.1) (width 0.25) (layer "F.Cu") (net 9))
 (segment (start 34.003903 37.613864) (end 35.041767 36.576) (width 0.25) (layer "F.Cu") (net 9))
 (segment (start 35.041767 36.576) (end 36.576 36.576) (width 0.25) (layer "F.Cu") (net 9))
 (segment (start 38.1 35.56) (end 35.35066 35.56) (width 0.25) (layer "F.Cu") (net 10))
 (segment (start 35.35066 35.56) (end 33.650349 37.260311) (width 0.25) (layer "F.Cu") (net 10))
 (segment (start 37.183553 33.02) (end 38.1 33.02) (width 0.25) (layer "F.Cu") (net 11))
 (segment (start 33.296796 36.906757) (end 37.183553 33.02) (width 0.25) (layer "F.Cu") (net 11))
 (segment (start 38.1 30.48) (end 36.925 31.655) (width 0.25) (layer "F.Cu") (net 12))
 (segment (start 36.925 32.571447) (end 32.943243 36.553204) (width 0.25) (layer "F.Cu") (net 12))
 (segment (start 36.925 31.655) (end 36.925 32.571447) (width 0.25) (layer "F.Cu") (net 12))
 (segment (start 36.009501 32.779839) (end 36.009501 30.030499) (width 0.25) (layer "F.Cu") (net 13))
 (segment (start 36.009501 30.030499) (end 38.1 27.94) (width 0.25) (layer "F.Cu") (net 13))
 (segment (start 32.589689 36.199651) (end 36.009501 32.779839) (width 0.25) (layer "F.Cu") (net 13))
 (segment (start 38.1 25.4) (end 35.56 27.94) (width 0.25) (layer "F.Cu") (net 14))
 (segment (start 35.56 32.522233) (end 32.236136 35.846097) (width 0.25) (layer "F.Cu") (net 14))
 (segment (start 35.56 27.94) (end 35.56 32.522233) (width 0.25) (layer "F.Cu") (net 14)))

